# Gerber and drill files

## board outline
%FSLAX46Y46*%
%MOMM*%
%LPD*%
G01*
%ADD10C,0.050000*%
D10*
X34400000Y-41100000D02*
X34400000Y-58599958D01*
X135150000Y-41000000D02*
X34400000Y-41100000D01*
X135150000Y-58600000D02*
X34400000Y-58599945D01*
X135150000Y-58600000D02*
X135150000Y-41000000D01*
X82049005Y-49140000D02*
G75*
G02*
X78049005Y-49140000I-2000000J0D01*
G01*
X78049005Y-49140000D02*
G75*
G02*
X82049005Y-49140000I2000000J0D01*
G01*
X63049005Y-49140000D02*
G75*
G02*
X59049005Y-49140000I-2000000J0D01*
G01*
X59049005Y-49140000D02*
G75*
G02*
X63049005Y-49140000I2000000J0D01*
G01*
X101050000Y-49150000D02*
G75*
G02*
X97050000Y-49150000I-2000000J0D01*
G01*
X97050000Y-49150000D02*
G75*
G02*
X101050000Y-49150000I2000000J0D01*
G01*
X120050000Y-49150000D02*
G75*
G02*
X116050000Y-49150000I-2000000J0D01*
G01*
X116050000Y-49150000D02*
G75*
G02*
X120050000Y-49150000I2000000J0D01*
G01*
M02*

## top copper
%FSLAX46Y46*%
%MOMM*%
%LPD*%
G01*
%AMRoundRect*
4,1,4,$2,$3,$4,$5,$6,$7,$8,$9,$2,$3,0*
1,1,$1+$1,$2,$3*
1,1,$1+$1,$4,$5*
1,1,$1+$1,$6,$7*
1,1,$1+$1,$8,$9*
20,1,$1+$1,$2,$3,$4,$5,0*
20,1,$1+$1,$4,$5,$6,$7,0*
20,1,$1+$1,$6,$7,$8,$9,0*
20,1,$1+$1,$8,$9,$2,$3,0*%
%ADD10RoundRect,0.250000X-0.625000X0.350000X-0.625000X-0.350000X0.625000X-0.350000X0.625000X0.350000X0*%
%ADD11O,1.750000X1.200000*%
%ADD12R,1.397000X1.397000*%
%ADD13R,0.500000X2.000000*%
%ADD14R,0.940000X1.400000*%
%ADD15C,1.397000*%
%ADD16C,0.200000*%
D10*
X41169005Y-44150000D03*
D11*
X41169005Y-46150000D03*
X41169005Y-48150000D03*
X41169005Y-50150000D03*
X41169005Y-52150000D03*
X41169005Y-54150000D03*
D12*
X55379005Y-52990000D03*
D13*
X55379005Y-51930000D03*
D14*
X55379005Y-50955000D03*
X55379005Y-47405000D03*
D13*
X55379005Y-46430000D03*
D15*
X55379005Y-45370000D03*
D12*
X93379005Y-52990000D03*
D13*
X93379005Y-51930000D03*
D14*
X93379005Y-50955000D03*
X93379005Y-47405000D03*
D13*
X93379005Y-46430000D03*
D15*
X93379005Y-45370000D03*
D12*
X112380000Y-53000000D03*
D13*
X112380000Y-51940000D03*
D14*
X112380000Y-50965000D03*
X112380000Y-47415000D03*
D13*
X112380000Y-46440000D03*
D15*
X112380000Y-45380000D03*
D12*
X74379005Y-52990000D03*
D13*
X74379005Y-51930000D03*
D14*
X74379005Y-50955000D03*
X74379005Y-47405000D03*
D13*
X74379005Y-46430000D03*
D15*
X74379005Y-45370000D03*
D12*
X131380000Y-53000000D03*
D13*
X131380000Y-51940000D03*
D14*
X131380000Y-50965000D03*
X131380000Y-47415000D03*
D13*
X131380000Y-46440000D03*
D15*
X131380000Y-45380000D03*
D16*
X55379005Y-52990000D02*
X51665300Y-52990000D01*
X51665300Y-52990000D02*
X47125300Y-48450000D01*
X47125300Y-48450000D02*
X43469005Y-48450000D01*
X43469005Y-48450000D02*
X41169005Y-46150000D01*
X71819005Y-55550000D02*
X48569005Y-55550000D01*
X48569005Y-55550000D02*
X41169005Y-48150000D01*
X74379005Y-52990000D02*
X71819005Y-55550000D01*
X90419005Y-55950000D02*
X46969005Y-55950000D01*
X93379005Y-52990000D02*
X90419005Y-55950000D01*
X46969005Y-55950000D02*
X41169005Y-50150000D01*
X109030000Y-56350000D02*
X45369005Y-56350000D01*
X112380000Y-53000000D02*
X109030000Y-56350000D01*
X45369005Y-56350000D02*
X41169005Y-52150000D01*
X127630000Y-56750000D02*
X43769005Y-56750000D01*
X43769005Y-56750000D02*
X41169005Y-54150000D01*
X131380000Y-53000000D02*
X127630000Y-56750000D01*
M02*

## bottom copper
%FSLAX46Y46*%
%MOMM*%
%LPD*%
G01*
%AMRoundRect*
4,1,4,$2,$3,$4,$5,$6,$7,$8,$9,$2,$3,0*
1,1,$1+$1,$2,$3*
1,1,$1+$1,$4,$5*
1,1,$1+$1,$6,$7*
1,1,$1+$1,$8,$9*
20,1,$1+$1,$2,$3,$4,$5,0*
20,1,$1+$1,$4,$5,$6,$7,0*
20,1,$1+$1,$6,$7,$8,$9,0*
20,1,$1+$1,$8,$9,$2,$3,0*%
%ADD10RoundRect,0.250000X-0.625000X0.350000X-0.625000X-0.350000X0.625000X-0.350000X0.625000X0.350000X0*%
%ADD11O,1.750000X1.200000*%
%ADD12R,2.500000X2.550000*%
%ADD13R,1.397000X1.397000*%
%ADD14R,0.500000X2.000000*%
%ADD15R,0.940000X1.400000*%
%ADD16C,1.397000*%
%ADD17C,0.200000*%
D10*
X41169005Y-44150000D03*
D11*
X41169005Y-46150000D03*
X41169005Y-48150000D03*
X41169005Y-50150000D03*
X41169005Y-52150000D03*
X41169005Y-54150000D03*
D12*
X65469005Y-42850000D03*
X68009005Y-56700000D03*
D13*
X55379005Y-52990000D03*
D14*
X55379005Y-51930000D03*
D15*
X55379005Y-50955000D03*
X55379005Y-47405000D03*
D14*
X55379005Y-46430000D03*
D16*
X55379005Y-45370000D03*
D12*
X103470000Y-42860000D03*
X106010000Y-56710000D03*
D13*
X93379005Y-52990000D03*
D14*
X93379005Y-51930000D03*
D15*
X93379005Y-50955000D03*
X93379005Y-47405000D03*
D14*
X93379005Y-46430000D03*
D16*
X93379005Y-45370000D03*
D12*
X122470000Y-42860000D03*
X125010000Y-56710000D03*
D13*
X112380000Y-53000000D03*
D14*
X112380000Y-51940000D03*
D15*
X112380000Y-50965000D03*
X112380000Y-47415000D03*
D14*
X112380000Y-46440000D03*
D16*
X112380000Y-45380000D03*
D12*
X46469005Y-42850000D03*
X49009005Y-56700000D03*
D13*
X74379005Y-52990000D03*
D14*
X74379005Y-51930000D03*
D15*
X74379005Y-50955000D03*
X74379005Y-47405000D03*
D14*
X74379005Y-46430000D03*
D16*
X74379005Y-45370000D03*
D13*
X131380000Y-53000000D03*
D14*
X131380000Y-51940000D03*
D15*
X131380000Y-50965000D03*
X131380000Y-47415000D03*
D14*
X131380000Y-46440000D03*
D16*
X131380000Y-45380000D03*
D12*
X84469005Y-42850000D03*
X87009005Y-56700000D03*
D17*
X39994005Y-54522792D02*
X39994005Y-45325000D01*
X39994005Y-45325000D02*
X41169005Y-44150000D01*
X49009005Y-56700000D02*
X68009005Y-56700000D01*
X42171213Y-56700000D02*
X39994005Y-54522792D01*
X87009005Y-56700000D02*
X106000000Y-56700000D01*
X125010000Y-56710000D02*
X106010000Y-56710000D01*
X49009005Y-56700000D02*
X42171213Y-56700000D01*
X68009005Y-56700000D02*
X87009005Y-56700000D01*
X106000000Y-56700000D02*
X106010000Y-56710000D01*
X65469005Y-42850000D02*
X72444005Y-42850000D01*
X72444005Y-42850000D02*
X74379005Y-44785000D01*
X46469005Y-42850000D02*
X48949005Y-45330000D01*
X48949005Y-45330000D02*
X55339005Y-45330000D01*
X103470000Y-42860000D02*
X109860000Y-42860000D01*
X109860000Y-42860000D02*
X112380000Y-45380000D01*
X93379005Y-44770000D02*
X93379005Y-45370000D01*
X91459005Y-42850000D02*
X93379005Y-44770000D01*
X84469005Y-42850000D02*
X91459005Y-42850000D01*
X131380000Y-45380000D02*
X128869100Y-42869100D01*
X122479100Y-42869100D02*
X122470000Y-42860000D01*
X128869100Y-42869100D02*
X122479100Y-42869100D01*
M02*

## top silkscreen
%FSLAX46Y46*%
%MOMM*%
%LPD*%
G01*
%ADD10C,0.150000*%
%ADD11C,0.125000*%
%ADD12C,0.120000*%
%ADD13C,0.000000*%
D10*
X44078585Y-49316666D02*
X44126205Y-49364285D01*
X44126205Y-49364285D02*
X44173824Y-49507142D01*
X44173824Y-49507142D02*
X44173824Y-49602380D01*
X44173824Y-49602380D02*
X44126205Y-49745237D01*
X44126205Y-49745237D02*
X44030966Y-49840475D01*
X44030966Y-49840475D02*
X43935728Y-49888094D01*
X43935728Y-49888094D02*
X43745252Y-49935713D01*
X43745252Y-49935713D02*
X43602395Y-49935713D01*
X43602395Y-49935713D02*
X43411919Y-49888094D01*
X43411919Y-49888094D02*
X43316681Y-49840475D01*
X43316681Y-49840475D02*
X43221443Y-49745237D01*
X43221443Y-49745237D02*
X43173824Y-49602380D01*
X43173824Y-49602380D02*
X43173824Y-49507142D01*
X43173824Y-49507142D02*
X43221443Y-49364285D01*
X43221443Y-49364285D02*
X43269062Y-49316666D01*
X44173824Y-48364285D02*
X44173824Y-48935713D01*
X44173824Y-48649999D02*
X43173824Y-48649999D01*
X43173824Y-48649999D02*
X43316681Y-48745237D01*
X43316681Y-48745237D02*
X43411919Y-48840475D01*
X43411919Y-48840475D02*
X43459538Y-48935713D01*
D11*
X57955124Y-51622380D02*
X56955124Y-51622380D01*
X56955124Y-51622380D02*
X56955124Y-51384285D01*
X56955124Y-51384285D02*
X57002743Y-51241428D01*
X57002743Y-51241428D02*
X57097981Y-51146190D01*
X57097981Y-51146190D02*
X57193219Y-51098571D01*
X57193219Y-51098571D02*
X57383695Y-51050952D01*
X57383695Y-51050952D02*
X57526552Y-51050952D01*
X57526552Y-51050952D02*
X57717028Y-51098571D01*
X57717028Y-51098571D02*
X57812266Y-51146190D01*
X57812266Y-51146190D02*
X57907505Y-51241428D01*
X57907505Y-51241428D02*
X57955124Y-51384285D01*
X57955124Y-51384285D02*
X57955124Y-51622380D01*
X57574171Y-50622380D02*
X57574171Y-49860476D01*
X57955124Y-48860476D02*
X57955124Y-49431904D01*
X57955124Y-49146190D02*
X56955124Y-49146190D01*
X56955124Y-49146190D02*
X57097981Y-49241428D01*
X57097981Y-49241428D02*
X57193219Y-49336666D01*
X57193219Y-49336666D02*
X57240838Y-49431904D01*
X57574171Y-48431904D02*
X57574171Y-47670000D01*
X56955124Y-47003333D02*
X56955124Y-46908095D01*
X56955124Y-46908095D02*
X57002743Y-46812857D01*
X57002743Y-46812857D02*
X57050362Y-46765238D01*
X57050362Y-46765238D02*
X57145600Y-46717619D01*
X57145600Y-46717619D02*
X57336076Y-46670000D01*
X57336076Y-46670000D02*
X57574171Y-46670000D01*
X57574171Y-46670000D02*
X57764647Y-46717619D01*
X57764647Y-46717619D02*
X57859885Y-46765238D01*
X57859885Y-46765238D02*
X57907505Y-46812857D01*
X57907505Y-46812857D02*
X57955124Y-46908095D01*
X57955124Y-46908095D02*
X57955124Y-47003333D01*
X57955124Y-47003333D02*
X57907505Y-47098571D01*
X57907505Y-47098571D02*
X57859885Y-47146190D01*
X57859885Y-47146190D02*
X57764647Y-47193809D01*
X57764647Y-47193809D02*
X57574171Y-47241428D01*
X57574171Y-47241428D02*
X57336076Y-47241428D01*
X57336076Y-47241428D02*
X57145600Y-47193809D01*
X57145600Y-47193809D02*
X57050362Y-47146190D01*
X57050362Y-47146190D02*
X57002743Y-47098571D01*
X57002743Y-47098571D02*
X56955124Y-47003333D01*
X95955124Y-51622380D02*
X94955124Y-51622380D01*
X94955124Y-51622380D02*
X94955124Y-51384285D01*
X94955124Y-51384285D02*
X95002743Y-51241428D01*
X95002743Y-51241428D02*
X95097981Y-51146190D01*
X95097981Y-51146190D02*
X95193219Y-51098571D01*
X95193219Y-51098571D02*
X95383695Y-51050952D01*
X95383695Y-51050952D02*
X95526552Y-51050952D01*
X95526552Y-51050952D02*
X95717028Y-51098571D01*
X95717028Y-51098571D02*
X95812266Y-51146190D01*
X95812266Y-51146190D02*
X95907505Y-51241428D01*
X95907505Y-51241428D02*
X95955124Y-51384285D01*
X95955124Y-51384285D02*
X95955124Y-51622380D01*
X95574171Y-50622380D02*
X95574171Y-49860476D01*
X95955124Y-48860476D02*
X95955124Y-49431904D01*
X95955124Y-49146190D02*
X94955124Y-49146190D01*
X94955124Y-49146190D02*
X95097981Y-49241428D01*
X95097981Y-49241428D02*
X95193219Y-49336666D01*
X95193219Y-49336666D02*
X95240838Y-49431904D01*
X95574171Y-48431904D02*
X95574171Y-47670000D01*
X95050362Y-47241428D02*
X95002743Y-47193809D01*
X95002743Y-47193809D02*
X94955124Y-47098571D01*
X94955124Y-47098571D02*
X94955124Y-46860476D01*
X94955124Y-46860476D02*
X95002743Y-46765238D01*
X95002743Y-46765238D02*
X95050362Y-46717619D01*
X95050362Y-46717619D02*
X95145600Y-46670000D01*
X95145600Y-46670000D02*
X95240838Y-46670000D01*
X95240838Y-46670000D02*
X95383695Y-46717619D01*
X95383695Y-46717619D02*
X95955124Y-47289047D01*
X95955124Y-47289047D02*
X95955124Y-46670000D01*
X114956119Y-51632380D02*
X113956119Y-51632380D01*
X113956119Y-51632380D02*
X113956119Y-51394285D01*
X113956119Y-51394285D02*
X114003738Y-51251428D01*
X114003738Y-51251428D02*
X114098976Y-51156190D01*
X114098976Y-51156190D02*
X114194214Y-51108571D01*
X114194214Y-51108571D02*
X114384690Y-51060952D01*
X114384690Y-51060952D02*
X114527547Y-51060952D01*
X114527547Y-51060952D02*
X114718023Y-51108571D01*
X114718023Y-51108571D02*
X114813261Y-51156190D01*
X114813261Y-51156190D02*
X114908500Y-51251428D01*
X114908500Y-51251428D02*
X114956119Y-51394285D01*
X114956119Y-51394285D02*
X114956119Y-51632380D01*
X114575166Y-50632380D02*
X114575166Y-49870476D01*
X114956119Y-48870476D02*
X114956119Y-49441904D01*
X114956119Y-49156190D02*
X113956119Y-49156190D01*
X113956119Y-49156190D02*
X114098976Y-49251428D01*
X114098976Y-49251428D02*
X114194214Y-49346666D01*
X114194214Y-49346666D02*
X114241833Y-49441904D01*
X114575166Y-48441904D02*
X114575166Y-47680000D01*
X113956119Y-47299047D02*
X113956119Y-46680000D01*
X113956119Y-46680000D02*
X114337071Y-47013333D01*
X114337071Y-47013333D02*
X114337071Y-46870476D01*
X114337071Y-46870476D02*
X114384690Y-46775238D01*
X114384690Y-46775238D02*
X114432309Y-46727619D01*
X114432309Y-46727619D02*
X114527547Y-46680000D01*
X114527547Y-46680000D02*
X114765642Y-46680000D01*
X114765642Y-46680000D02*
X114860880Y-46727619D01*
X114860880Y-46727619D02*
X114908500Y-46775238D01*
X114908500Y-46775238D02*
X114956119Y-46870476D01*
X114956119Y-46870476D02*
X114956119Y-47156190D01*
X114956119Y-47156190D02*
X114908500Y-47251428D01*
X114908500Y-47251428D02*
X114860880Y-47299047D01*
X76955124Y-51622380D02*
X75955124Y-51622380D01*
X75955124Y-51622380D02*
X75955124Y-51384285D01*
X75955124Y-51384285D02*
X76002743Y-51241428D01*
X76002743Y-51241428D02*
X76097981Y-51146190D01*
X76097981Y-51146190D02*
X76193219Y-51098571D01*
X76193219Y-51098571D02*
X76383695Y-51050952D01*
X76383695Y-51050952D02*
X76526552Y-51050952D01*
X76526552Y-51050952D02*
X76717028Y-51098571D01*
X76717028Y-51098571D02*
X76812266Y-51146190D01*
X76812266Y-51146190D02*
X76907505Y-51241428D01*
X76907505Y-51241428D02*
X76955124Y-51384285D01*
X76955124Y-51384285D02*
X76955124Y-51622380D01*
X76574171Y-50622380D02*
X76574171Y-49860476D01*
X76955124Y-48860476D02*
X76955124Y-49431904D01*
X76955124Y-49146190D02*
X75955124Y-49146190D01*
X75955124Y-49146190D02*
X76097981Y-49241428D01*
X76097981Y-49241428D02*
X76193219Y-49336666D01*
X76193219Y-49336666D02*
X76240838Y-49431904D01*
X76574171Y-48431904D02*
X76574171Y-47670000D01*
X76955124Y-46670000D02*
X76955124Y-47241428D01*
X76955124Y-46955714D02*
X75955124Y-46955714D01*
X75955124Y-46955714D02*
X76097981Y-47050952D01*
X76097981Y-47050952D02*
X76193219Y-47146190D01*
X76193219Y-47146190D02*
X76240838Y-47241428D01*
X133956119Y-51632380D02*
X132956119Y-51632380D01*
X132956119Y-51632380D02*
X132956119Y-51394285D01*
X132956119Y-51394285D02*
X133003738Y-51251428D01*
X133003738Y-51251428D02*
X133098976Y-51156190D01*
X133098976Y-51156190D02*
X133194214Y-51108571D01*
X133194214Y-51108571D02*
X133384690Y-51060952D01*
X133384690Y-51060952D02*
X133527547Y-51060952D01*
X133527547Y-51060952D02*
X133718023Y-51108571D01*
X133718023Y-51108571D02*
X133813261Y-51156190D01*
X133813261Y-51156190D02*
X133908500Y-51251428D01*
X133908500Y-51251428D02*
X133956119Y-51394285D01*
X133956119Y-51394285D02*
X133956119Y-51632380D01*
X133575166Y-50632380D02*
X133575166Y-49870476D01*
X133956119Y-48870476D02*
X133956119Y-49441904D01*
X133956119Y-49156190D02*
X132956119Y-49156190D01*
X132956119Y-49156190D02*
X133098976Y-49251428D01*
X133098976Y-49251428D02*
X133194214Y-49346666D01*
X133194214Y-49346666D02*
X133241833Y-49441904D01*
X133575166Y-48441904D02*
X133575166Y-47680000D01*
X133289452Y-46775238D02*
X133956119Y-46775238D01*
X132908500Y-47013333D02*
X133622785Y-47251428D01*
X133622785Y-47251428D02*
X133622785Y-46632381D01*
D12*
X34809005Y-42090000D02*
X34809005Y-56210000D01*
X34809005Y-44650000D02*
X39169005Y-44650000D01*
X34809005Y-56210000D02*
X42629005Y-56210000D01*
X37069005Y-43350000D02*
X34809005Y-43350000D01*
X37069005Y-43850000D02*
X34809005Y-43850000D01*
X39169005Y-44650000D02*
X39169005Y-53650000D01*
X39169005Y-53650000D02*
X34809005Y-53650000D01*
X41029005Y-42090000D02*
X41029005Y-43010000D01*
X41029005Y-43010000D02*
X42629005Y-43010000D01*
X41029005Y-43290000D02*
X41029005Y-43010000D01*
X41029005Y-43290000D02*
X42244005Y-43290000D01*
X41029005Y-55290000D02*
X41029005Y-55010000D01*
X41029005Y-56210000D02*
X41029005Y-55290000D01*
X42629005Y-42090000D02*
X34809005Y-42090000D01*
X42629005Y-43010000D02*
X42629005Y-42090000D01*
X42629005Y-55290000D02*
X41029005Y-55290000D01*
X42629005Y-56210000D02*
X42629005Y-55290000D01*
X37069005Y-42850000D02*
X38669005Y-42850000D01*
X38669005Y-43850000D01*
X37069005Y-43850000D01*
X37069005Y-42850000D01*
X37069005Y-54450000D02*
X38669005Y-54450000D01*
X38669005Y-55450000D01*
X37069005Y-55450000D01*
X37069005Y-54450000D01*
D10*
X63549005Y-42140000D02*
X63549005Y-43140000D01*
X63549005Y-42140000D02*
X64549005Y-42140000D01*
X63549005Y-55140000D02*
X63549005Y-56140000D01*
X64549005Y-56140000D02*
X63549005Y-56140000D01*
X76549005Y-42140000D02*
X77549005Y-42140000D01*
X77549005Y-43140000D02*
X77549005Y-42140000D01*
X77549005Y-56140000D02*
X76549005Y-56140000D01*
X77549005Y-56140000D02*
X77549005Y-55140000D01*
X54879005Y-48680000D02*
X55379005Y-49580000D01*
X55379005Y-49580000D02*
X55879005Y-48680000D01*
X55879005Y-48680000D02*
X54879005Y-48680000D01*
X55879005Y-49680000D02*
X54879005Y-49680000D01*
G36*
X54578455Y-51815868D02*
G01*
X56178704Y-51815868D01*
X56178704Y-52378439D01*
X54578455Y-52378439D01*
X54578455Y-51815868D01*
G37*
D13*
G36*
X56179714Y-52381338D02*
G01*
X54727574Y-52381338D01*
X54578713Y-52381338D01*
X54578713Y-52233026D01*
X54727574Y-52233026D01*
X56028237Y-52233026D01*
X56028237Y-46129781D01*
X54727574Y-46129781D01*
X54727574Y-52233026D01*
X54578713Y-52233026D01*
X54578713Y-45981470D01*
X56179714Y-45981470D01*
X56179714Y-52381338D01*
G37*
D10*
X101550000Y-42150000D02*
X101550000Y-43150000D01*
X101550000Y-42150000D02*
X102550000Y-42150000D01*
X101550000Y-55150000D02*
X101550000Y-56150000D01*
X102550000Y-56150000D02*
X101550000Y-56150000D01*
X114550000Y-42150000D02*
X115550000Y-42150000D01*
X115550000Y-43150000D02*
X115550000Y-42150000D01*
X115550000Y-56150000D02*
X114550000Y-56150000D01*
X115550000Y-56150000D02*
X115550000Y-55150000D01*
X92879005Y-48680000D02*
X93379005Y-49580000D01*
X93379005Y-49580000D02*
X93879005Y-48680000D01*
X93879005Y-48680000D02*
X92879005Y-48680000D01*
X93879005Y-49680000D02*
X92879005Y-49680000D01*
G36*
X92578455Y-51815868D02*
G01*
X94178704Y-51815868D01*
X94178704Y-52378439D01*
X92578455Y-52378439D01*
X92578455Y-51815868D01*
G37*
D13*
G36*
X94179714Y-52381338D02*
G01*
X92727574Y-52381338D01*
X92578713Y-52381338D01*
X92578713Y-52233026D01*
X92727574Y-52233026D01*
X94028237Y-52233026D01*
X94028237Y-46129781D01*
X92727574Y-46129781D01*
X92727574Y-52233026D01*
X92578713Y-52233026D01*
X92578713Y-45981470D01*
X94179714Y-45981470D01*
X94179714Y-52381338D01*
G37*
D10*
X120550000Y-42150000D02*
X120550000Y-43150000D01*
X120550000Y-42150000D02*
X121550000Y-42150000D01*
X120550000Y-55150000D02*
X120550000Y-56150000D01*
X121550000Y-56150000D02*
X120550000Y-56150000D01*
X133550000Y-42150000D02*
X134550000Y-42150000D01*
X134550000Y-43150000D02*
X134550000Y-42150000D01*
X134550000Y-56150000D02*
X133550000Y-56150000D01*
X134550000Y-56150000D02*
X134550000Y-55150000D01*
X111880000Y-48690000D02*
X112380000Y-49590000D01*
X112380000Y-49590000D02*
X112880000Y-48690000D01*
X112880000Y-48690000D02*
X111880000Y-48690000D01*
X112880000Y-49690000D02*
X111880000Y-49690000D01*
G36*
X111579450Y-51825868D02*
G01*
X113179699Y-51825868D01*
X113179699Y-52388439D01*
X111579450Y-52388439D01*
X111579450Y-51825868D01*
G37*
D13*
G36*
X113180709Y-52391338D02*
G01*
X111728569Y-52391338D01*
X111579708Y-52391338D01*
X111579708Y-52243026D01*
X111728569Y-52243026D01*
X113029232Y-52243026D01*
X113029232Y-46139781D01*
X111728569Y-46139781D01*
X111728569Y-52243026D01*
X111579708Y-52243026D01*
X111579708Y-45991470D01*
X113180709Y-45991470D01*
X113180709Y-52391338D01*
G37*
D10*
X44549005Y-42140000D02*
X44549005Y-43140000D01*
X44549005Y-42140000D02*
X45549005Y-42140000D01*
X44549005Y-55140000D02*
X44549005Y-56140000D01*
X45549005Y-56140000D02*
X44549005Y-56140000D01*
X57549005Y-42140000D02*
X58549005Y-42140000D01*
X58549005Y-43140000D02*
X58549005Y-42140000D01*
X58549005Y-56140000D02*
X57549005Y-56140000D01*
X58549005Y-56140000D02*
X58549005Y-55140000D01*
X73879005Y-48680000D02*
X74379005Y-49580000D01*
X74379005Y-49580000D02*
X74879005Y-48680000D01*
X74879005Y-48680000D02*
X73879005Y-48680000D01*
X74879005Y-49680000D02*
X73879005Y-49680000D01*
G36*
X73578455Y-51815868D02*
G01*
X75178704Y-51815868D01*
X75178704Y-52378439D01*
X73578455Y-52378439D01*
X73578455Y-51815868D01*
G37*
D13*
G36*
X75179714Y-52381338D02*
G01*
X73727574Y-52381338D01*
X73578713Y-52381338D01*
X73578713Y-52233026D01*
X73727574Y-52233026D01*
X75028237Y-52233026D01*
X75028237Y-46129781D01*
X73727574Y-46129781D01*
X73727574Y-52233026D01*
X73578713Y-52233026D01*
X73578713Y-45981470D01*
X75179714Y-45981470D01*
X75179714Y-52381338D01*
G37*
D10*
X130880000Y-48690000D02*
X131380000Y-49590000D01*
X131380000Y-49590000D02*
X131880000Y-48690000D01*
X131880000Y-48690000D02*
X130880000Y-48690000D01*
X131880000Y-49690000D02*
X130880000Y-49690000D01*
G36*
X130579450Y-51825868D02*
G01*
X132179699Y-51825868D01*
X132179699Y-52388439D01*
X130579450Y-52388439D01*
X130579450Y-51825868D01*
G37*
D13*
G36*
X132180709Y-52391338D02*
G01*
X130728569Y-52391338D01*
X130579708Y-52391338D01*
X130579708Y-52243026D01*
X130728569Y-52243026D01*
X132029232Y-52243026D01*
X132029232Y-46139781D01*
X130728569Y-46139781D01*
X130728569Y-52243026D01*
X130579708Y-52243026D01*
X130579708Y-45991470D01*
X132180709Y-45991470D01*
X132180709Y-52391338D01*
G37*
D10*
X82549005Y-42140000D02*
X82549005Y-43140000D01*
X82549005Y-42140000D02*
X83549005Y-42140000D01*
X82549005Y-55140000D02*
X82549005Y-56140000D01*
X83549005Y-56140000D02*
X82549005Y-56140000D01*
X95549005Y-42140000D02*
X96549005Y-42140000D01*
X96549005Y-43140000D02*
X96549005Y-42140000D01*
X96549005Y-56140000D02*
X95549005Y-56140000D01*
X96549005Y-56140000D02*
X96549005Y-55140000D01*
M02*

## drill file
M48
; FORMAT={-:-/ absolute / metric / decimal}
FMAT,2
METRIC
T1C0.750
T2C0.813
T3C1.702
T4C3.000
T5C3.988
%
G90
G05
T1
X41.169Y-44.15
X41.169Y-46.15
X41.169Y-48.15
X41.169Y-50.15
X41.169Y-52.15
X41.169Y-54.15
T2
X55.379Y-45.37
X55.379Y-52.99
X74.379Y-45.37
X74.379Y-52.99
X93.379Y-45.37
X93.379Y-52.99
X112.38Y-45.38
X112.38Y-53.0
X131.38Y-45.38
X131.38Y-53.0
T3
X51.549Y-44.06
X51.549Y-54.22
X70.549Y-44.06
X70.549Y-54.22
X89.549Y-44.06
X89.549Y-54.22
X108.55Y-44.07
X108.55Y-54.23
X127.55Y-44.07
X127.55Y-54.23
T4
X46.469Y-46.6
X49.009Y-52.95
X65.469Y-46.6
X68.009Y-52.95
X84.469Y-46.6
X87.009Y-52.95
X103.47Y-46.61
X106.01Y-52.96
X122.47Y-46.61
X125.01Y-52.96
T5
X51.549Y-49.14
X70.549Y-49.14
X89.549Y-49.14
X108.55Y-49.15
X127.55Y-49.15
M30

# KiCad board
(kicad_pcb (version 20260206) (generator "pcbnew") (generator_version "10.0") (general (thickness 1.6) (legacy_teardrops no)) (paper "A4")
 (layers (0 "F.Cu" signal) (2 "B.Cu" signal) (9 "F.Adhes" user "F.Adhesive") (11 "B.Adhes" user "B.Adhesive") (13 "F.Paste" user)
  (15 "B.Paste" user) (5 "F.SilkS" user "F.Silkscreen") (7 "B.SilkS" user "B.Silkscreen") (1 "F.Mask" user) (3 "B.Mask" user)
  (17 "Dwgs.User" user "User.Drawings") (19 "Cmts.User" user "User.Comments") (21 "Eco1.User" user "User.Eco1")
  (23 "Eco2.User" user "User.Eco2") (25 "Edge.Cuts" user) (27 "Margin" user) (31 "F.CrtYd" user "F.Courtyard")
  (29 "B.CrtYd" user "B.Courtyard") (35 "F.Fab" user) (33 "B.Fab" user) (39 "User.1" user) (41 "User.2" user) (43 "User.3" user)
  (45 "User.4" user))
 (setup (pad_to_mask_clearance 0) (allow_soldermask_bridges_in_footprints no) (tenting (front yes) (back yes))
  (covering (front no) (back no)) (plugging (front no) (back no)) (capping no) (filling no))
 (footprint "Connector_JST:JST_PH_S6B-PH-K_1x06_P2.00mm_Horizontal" (layer "F.Cu") (at 41.169005 44.15 -90)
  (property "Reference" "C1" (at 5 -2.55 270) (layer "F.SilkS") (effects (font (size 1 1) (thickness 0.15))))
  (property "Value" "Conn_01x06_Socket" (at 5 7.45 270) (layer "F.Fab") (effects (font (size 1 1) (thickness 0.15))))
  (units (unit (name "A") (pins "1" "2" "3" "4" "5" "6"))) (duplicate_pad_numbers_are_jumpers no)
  (fp_line (start -2.06 6.36) (end 12.06 6.36) (stroke (width 0.12) (type solid)) (layer "F.SilkS"))
  (fp_line (start 0.5 6.36) (end 0.5 2) (stroke (width 0.12) (type solid)) (layer "F.SilkS"))
  (fp_line (start 12.06 6.36) (end 12.06 -1.46) (stroke (width 0.12) (type solid)) (layer "F.SilkS"))
  (fp_line (start -0.8 4.1) (end -0.8 6.36) (stroke (width 0.12) (type solid)) (layer "F.SilkS"))
  (fp_line (start -0.3 4.1) (end -0.3 6.36) (stroke (width 0.12) (type solid)) (layer "F.SilkS"))
  (fp_line (start 0.5 2) (end 9.5 2) (stroke (width 0.12) (type solid)) (layer "F.SilkS"))
  (fp_line (start 9.5 2) (end 9.5 6.36) (stroke (width 0.12) (type solid)) (layer "F.SilkS"))
  (fp_line (start -2.06 0.14) (end -1.14 0.14) (stroke (width 0.12) (type solid)) (layer "F.SilkS"))
  (fp_line (start -1.14 0.14) (end -1.14 -1.46) (stroke (width 0.12) (type solid)) (layer "F.SilkS"))
  (fp_line (start -0.86 0.14) (end -1.14 0.14) (stroke (width 0.12) (type solid)) (layer "F.SilkS"))
  (fp_line (start -0.86 0.14) (end -0.86 -1.075) (stroke (width 0.12) (type solid)) (layer "F.SilkS"))
  (fp_line (start 11.14 0.14) (end 10.86 0.14) (stroke (width 0.12) (type solid)) (layer "F.SilkS"))
  (fp_line (start 12.06 0.14) (end 11.14 0.14) (stroke (width 0.12) (type solid)) (layer "F.SilkS"))
  (fp_line (start -2.06 -1.46) (end -2.06 6.36) (stroke (width 0.12) (type solid)) (layer "F.SilkS"))
  (fp_line (start -1.14 -1.46) (end -2.06 -1.46) (stroke (width 0.12) (type solid)) (layer "F.SilkS"))
  (fp_line (start 11.14 -1.46) (end 11.14 0.14) (stroke (width 0.12) (type solid)) (layer "F.SilkS"))
  (fp_line (start 12.06 -1.46) (end 11.14 -1.46) (stroke (width 0.12) (type solid)) (layer "F.SilkS"))
  (fp_rect (start -1.3 2.5) (end -0.3 4.1) (stroke (width 0.12) (type solid)) (fill no) (layer "F.SilkS"))
  (fp_rect (start 10.3 2.5) (end 11.3 4.1) (stroke (width 0.12) (type solid)) (fill no) (layer "F.SilkS"))
  (pad "1" thru_hole roundrect (at 0 0 270) (size 1.2 1.75) (drill 0.75) (layers "*.Cu" "*.Mask") (remove_unused_layers no)
   (roundrect_rratio 0.208333) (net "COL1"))
  (pad "2" thru_hole oval (at 2 0 270) (size 1.2 1.75) (drill 0.75) (layers "*.Cu" "*.Mask") (remove_unused_layers no) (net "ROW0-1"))
  (pad "3" thru_hole oval (at 4 0 270) (size 1.2 1.75) (drill 0.75) (layers "*.Cu" "*.Mask") (remove_unused_layers no) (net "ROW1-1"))
  (pad "4" thru_hole oval (at 6 0 270) (size 1.2 1.75) (drill 0.75) (layers "*.Cu" "*.Mask") (remove_unused_layers no) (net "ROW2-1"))
  (pad "5" thru_hole oval (at 8 0 270) (size 1.2 1.75) (drill 0.75) (layers "*.Cu" "*.Mask") (remove_unused_layers no) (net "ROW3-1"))
  (pad "6" thru_hole oval (at 10 0 270) (size 1.2 1.75) (drill 0.75) (layers "*.Cu" "*.Mask") (remove_unused_layers no) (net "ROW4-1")))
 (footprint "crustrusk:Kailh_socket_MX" (layer "F.Cu") (at 70.549005 49.14 90)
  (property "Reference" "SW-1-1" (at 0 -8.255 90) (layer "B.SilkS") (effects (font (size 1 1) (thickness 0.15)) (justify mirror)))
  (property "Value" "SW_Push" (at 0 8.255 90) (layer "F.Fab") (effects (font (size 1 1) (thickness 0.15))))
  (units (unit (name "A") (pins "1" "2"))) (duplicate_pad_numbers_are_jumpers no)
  (fp_line (start 7 -7) (end 6 -7) (stroke (width 0.15) (type solid)) (layer "F.SilkS"))
  (fp_line (start 7 -7) (end 7 -6) (stroke (width 0.15) (type solid)) (layer "F.SilkS"))
  (fp_line (start -6 -7) (end -7 -7) (stroke (width 0.15) (type solid)) (layer "F.SilkS"))
  (fp_line (start -7 -6) (end -7 -7) (stroke (width 0.15) (type solid)) (layer "F.SilkS"))
  (fp_line (start 7 6) (end 7 7) (stroke (width 0.15) (type solid)) (layer "F.SilkS"))
  (fp_line (start 6 7) (end 7 7) (stroke (width 0.15) (type solid)) (layer "F.SilkS"))
  (fp_line (start -7 7) (end -7 6) (stroke (width 0.15) (type solid)) (layer "F.SilkS"))
  (fp_line (start -7 7) (end -6 7) (stroke (width 0.15) (type solid)) (layer "F.SilkS"))
  (pad "" np_thru_hole circle (at -5.08 0 90) (size 1.7018 1.7018) (drill 1.7018) (layers "*.Cu" "*.Mask"))
  (pad "" np_thru_hole circle (at -3.81 -2.54 90) (size 3 3) (drill 3) (layers "*.Cu" "*.Mask"))
  (pad "" np_thru_hole circle (at 0 0 90) (size 3.9878 3.9878) (drill 3.9878) (layers "*.Cu" "*.Mask"))
  (pad "" np_thru_hole circle (at 2.54 -5.08 90) (size 3 3) (drill 3) (layers "*.Cu" "*.Mask"))
  (pad "" np_thru_hole circle (at 5.08 0 90) (size 1.7018 1.7018) (drill 1.7018) (layers "*.Cu" "*.Mask"))
  (pad "1" smd rect (at 6.29 -5.08 90) (size 2.55 2.5) (layers "B.Cu" "B.Mask" "B.Paste") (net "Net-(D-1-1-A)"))
  (pad "2" smd rect (at -7.56 -2.54 90) (size 2.55 2.5) (layers "B.Cu" "B.Mask" "B.Paste") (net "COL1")))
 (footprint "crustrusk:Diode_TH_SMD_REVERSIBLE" (layer "F.Cu") (at 55.379005 49.18 90)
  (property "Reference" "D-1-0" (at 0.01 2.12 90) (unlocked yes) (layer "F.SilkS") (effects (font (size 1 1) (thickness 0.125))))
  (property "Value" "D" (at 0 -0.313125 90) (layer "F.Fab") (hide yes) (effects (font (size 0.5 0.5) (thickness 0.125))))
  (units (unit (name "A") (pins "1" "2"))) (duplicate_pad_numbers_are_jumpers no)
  (fp_line (start 0.5 -0.5) (end -0.4 0) (stroke (width 0.15) (type solid)) (layer "F.SilkS"))
  (fp_line (start -0.4 0) (end 0.5 0.5) (stroke (width 0.15) (type solid)) (layer "F.SilkS"))
  (fp_line (start 0.5 0.5) (end 0.5 -0.5) (stroke (width 0.15) (type solid)) (layer "F.SilkS"))
  (fp_line (start -0.5 0.5) (end -0.5 -0.5) (stroke (width 0.15) (type solid)) (layer "F.SilkS"))
  (fp_rect (start -3.198439 -0.80055) (end -2.635868 0.799699) (stroke (width -0.000001) (type solid)) (fill yes) (layer "F.SilkS"))
  (fp_poly
   (pts (xy 3.19853 -0.800292) (xy -3.201338 -0.800292) (xy -3.201338 -0.651431) (xy -3.053026 -0.651431) (xy 3.050219 -0.651431)
    (xy 3.050219 0.649232) (xy -3.053026 0.649232) (xy -3.053026 -0.651431) (xy -3.201338 -0.651431) (xy -3.201338 0.800709)
    (xy 3.19853 0.800709))
   (stroke (width -0.000001) (type solid)) (fill yes) (layer "F.SilkS"))
  (pad "1" thru_hole rect (at -3.81 0 90) (size 1.397 1.397) (drill 0.8128) (layers "*.Cu" "*.Mask") (remove_unused_layers no)
   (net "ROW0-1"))
  (pad "1" smd rect (at -2.75 0 270) (size 2 0.5) (layers "F.Cu") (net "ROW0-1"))
  (pad "1" smd rect (at -2.75 0 90) (size 2 0.5) (layers "B.Cu") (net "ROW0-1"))
  (pad "1" smd rect (at -1.775 0 270) (size 1.4 0.94) (layers "F.Cu" "F.Mask" "F.Paste") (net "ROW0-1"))
  (pad "1" smd rect (at -1.775 0 90) (size 1.4 0.94) (layers "B.Cu" "B.Mask" "B.Paste") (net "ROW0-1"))
  (pad "2" smd rect (at 1.775 0 270) (size 1.4 0.94) (layers "F.Cu" "F.Mask" "F.Paste") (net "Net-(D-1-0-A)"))
  (pad "2" smd rect (at 1.775 0 90) (size 1.4 0.94) (layers "B.Cu" "B.Mask" "B.Paste") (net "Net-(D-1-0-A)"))
  (pad "2" smd rect (at 2.75 0 270) (size 2 0.5) (layers "F.Cu") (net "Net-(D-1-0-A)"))
  (pad "2" smd rect (at 2.75 0 90) (size 2 0.5) (layers "B.Cu") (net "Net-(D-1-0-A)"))
  (pad "2" thru_hole circle (at 3.81 0 90) (size 1.397 1.397) (drill 0.8128) (layers "*.Cu" "*.Mask") (remove_unused_layers no)
   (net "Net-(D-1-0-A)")))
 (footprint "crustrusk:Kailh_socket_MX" (layer "F.Cu") (at 108.55 49.15 90)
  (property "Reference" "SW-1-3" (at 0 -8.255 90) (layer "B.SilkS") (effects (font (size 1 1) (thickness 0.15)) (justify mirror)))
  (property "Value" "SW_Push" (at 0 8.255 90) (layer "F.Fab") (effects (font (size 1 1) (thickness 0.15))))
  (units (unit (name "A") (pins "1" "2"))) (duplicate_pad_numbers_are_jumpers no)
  (fp_line (start 7 -7) (end 6 -7) (stroke (width 0.15) (type solid)) (layer "F.SilkS"))
  (fp_line (start 7 -7) (end 7 -6) (stroke (width 0.15) (type solid)) (layer "F.SilkS"))
  (fp_line (start -6 -7) (end -7 -7) (stroke (width 0.15) (type solid)) (layer "F.SilkS"))
  (fp_line (start -7 -6) (end -7 -7) (stroke (width 0.15) (type solid)) (layer "F.SilkS"))
  (fp_line (start 7 6) (end 7 7) (stroke (width 0.15) (type solid)) (layer "F.SilkS"))
  (fp_line (start 6 7) (end 7 7) (stroke (width 0.15) (type solid)) (layer "F.SilkS"))
  (fp_line (start -7 7) (end -7 6) (stroke (width 0.15) (type solid)) (layer "F.SilkS"))
  (fp_line (start -7 7) (end -6 7) (stroke (width 0.15) (type solid)) (layer "F.SilkS"))
  (pad "" np_thru_hole circle (at -5.08 0 90) (size 1.7018 1.7018) (drill 1.7018) (layers "*.Cu" "*.Mask"))
  (pad "" np_thru_hole circle (at -3.81 -2.54 90) (size 3 3) (drill 3) (layers "*.Cu" "*.Mask"))
  (pad "" np_thru_hole circle (at 0 0 90) (size 3.9878 3.9878) (drill 3.9878) (layers "*.Cu" "*.Mask"))
  (pad "" np_thru_hole circle (at 2.54 -5.08 90) (size 3 3) (drill 3) (layers "*.Cu" "*.Mask"))
  (pad "" np_thru_hole circle (at 5.08 0 90) (size 1.7018 1.7018) (drill 1.7018) (layers "*.Cu" "*.Mask"))
  (pad "1" smd rect (at 6.29 -5.08 90) (size 2.55 2.5) (layers "B.Cu" "B.Mask" "B.Paste") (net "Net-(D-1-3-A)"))
  (pad "2" smd rect (at -7.56 -2.54 90) (size 2.55 2.5) (layers "B.Cu" "B.Mask" "B.Paste") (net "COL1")))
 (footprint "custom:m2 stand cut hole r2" (layer "F.Cu") (at 80.049005 49.14 90)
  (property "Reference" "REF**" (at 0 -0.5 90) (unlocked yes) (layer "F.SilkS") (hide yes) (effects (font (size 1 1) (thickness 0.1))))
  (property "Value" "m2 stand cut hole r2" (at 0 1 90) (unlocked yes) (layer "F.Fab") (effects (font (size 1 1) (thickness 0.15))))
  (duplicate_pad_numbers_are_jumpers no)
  (fp_circle (center 0 0) (end 2 0) (stroke (width 0.05) (type default)) (fill no) (layer "Edge.Cuts")))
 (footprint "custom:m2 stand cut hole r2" (layer "F.Cu") (at 61.049005 49.14 90)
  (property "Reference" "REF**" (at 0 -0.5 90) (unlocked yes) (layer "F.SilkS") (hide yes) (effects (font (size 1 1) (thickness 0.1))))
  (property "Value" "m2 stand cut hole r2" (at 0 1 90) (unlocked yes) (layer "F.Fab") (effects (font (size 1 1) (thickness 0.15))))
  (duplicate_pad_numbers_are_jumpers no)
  (fp_circle (center 0 0) (end 2 0) (stroke (width 0.05) (type default)) (fill no) (layer "Edge.Cuts")))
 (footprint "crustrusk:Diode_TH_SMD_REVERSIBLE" (layer "F.Cu") (at 93.379005 49.18 90)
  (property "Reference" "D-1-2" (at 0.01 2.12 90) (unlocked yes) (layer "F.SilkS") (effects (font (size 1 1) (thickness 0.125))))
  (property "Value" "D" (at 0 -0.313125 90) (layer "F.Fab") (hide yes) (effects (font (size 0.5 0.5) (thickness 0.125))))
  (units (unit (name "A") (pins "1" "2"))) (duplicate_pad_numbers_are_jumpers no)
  (fp_line (start 0.5 -0.5) (end -0.4 0) (stroke (width 0.15) (type solid)) (layer "F.SilkS"))
  (fp_line (start -0.4 0) (end 0.5 0.5) (stroke (width 0.15) (type solid)) (layer "F.SilkS"))
  (fp_line (start 0.5 0.5) (end 0.5 -0.5) (stroke (width 0.15) (type solid)) (layer "F.SilkS"))
  (fp_line (start -0.5 0.5) (end -0.5 -0.5) (stroke (width 0.15) (type solid)) (layer "F.SilkS"))
  (fp_rect (start -3.198439 -0.80055) (end -2.635868 0.799699) (stroke (width -0.000001) (type solid)) (fill yes) (layer "F.SilkS"))
  (fp_poly
   (pts (xy 3.19853 -0.800292) (xy -3.201338 -0.800292) (xy -3.201338 -0.651431) (xy -3.053026 -0.651431) (xy 3.050219 -0.651431)
    (xy 3.050219 0.649232) (xy -3.053026 0.649232) (xy -3.053026 -0.651431) (xy -3.201338 -0.651431) (xy -3.201338 0.800709)
    (xy 3.19853 0.800709))
   (stroke (width -0.000001) (type solid)) (fill yes) (layer "F.SilkS"))
  (pad "1" thru_hole rect (at -3.81 0 90) (size 1.397 1.397) (drill 0.8128) (layers "*.Cu" "*.Mask") (remove_unused_layers no)
   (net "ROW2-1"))
  (pad "1" smd rect (at -2.75 0 270) (size 2 0.5) (layers "F.Cu") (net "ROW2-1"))
  (pad "1" smd rect (at -2.75 0 90) (size 2 0.5) (layers "B.Cu") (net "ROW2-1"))
  (pad "1" smd rect (at -1.775 0 270) (size 1.4 0.94) (layers "F.Cu" "F.Mask" "F.Paste") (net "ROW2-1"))
  (pad "1" smd rect (at -1.775 0 90) (size 1.4 0.94) (layers "B.Cu" "B.Mask" "B.Paste") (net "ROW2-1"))
  (pad "2" smd rect (at 1.775 0 270) (size 1.4 0.94) (layers "F.Cu" "F.Mask" "F.Paste") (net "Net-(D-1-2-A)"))
  (pad "2" smd rect (at 1.775 0 90) (size 1.4 0.94) (layers "B.Cu" "B.Mask" "B.Paste") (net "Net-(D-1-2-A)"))
  (pad "2" smd rect (at 2.75 0 270) (size 2 0.5) (layers "F.Cu") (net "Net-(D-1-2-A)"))
  (pad "2" smd rect (at 2.75 0 90) (size 2 0.5) (layers "B.Cu") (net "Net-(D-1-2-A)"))
  (pad "2" thru_hole circle (at 3.81 0 90) (size 1.397 1.397) (drill 0.8128) (layers "*.Cu" "*.Mask") (remove_unused_layers no)
   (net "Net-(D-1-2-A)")))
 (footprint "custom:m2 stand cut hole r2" (layer "F.Cu") (at 99.05 49.15 90)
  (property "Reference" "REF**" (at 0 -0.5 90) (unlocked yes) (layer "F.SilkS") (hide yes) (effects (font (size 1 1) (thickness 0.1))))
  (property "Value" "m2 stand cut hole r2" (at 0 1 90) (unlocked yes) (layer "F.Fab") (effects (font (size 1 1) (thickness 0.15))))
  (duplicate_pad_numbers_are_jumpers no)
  (fp_circle (center 0 0) (end 2 0) (stroke (width 0.05) (type default)) (fill no) (layer "Edge.Cuts")))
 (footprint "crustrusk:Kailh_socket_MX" (layer "F.Cu") (at 127.55 49.15 90)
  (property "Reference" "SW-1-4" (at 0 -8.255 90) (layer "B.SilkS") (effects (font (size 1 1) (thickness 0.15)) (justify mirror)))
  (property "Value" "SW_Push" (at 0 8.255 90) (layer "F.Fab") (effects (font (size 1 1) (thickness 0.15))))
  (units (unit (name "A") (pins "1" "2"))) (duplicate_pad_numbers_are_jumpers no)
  (fp_line (start 7 -7) (end 6 -7) (stroke (width 0.15) (type solid)) (layer "F.SilkS"))
  (fp_line (start 7 -7) (end 7 -6) (stroke (width 0.15) (type solid)) (layer "F.SilkS"))
  (fp_line (start -6 -7) (end -7 -7) (stroke (width 0.15) (type solid)) (layer "F.SilkS"))
  (fp_line (start -7 -6) (end -7 -7) (stroke (width 0.15) (type solid)) (layer "F.SilkS"))
  (fp_line (start 7 6) (end 7 7) (stroke (width 0.15) (type solid)) (layer "F.SilkS"))
  (fp_line (start 6 7) (end 7 7) (stroke (width 0.15) (type solid)) (layer "F.SilkS"))
  (fp_line (start -7 7) (end -7 6) (stroke (width 0.15) (type solid)) (layer "F.SilkS"))
  (fp_line (start -7 7) (end -6 7) (stroke (width 0.15) (type solid)) (layer "F.SilkS"))
  (pad "" np_thru_hole circle (at -5.08 0 90) (size 1.7018 1.7018) (drill 1.7018) (layers "*.Cu" "*.Mask"))
  (pad "" np_thru_hole circle (at -3.81 -2.54 90) (size 3 3) (drill 3) (layers "*.Cu" "*.Mask"))
  (pad "" np_thru_hole circle (at 0 0 90) (size 3.9878 3.9878) (drill 3.9878) (layers "*.Cu" "*.Mask"))
  (pad "" np_thru_hole circle (at 2.54 -5.08 90) (size 3 3) (drill 3) (layers "*.Cu" "*.Mask"))
  (pad "" np_thru_hole circle (at 5.08 0 90) (size 1.7018 1.7018) (drill 1.7018) (layers "*.Cu" "*.Mask"))
  (pad "1" smd rect (at 6.29 -5.08 90) (size 2.55 2.5) (layers "B.Cu" "B.Mask" "B.Paste") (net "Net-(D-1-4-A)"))
  (pad "2" smd rect (at -7.56 -2.54 90) (size 2.55 2.5) (layers "B.Cu" "B.Mask" "B.Paste") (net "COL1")))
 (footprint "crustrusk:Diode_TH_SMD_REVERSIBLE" (layer "F.Cu") (at 112.38 49.19 90)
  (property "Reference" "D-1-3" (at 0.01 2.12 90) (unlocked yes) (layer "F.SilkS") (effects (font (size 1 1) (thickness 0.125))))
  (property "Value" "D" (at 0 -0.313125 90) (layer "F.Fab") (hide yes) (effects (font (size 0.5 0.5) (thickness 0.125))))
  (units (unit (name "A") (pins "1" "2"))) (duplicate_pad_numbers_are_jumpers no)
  (fp_line (start 0.5 -0.5) (end -0.4 0) (stroke (width 0.15) (type solid)) (layer "F.SilkS"))
  (fp_line (start -0.4 0) (end 0.5 0.5) (stroke (width 0.15) (type solid)) (layer "F.SilkS"))
  (fp_line (start 0.5 0.5) (end 0.5 -0.5) (stroke (width 0.15) (type solid)) (layer "F.SilkS"))
  (fp_line (start -0.5 0.5) (end -0.5 -0.5) (stroke (width 0.15) (type solid)) (layer "F.SilkS"))
  (fp_rect (start -3.198439 -0.80055) (end -2.635868 0.799699) (stroke (width -0.000001) (type solid)) (fill yes) (layer "F.SilkS"))
  (fp_poly
   (pts (xy 3.19853 -0.800292) (xy -3.201338 -0.800292) (xy -3.201338 -0.651431) (xy -3.053026 -0.651431) (xy 3.050219 -0.651431)
    (xy 3.050219 0.649232) (xy -3.053026 0.649232) (xy -3.053026 -0.651431) (xy -3.201338 -0.651431) (xy -3.201338 0.800709)
    (xy 3.19853 0.800709))
   (stroke (width -0.000001) (type solid)) (fill yes) (layer "F.SilkS"))
  (pad "1" thru_hole rect (at -3.81 0 90) (size 1.397 1.397) (drill 0.8128) (layers "*.Cu" "*.Mask") (remove_unused_layers no)
   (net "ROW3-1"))
  (pad "1" smd rect (at -2.75 0 270) (size 2 0.5) (layers "F.Cu") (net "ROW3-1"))
  (pad "1" smd rect (at -2.75 0 90) (size 2 0.5) (layers "B.Cu") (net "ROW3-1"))
  (pad "1" smd rect (at -1.775 0 270) (size 1.4 0.94) (layers "F.Cu" "F.Mask" "F.Paste") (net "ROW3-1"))
  (pad "1" smd rect (at -1.775 0 90) (size 1.4 0.94) (layers "B.Cu" "B.Mask" "B.Paste") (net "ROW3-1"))
  (pad "2" smd rect (at 1.775 0 270) (size 1.4 0.94) (layers "F.Cu" "F.Mask" "F.Paste") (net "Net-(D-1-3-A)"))
  (pad "2" smd rect (at 1.775 0 90) (size 1.4 0.94) (layers "B.Cu" "B.Mask" "B.Paste") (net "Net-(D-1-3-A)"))
  (pad "2" smd rect (at 2.75 0 270) (size 2 0.5) (layers "F.Cu") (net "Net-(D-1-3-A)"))
  (pad "2" smd rect (at 2.75 0 90) (size 2 0.5) (layers "B.Cu") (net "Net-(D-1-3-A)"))
  (pad "2" thru_hole circle (at 3.81 0 90) (size 1.397 1.397) (drill 0.8128) (layers "*.Cu" "*.Mask") (remove_unused_layers no)
   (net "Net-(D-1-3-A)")))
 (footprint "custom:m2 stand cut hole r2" (layer "F.Cu") (at 118.05 49.15 90)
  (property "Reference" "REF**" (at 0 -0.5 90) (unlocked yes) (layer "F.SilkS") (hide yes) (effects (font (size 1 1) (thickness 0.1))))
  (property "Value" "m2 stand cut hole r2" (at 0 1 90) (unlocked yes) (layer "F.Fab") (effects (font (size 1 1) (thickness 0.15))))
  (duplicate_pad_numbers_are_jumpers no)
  (fp_circle (center 0 0) (end 2 0) (stroke (width 0.05) (type default)) (fill no) (layer "Edge.Cuts")))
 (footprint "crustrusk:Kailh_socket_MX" (layer "F.Cu") (at 51.549005 49.14 90)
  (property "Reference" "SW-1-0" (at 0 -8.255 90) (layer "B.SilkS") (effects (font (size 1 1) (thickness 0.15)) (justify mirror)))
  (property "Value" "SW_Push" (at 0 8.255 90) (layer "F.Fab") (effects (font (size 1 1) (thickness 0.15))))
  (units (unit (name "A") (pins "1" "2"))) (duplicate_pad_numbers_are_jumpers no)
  (fp_line (start 7 -7) (end 6 -7) (stroke (width 0.15) (type solid)) (layer "F.SilkS"))
  (fp_line (start 7 -7) (end 7 -6) (stroke (width 0.15) (type solid)) (layer "F.SilkS"))
  (fp_line (start -6 -7) (end -7 -7) (stroke (width 0.15) (type solid)) (layer "F.SilkS"))
  (fp_line (start -7 -6) (end -7 -7) (stroke (width 0.15) (type solid)) (layer "F.SilkS"))
  (fp_line (start 7 6) (end 7 7) (stroke (width 0.15) (type solid)) (layer "F.SilkS"))
  (fp_line (start 6 7) (end 7 7) (stroke (width 0.15) (type solid)) (layer "F.SilkS"))
  (fp_line (start -7 7) (end -7 6) (stroke (width 0.15) (type solid)) (layer "F.SilkS"))
  (fp_line (start -7 7) (end -6 7) (stroke (width 0.15) (type solid)) (layer "F.SilkS"))
  (pad "" np_thru_hole circle (at -5.08 0 90) (size 1.7018 1.7018) (drill 1.7018) (layers "*.Cu" "*.Mask"))
  (pad "" np_thru_hole circle (at -3.81 -2.54 90) (size 3 3) (drill 3) (layers "*.Cu" "*.Mask"))
  (pad "" np_thru_hole circle (at 0 0 90) (size 3.9878 3.9878) (drill 3.9878) (layers "*.Cu" "*.Mask"))
  (pad "" np_thru_hole circle (at 2.54 -5.08 90) (size 3 3) (drill 3) (layers "*.Cu" "*.Mask"))
  (pad "" np_thru_hole circle (at 5.08 0 90) (size 1.7018 1.7018) (drill 1.7018) (layers "*.Cu" "*.Mask"))
  (pad "1" smd rect (at 6.29 -5.08 90) (size 2.55 2.5) (layers "B.Cu" "B.Mask" "B.Paste") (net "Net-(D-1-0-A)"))
  (pad "2" smd rect (at -7.56 -2.54 90) (size 2.55 2.5) (layers "B.Cu" "B.Mask" "B.Paste") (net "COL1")))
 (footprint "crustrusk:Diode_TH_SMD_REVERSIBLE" (layer "F.Cu") (at 74.379005 49.18 90)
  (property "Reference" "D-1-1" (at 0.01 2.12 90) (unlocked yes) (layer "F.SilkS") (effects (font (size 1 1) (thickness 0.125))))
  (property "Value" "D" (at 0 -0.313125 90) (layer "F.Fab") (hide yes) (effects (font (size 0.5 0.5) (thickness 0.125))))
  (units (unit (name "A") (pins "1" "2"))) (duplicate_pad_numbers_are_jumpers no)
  (fp_line (start 0.5 -0.5) (end -0.4 0) (stroke (width 0.15) (type solid)) (layer "F.SilkS"))
  (fp_line (start -0.4 0) (end 0.5 0.5) (stroke (width 0.15) (type solid)) (layer "F.SilkS"))
  (fp_line (start 0.5 0.5) (end 0.5 -0.5) (stroke (width 0.15) (type solid)) (layer "F.SilkS"))
  (fp_line (start -0.5 0.5) (end -0.5 -0.5) (stroke (width 0.15) (type solid)) (layer "F.SilkS"))
  (fp_rect (start -3.198439 -0.80055) (end -2.635868 0.799699) (stroke (width -0.000001) (type solid)) (fill yes) (layer "F.SilkS"))
  (fp_poly
   (pts (xy 3.19853 -0.800292) (xy -3.201338 -0.800292) (xy -3.201338 -0.651431) (xy -3.053026 -0.651431) (xy 3.050219 -0.651431)
    (xy 3.050219 0.649232) (xy -3.053026 0.649232) (xy -3.053026 -0.651431) (xy -3.201338 -0.651431) (xy -3.201338 0.800709)
    (xy 3.19853 0.800709))
   (stroke (width -0.000001) (type solid)) (fill yes) (layer "F.SilkS"))
  (pad "1" thru_hole rect (at -3.81 0 90) (size 1.397 1.397) (drill 0.8128) (layers "*.Cu" "*.Mask") (remove_unused_layers no)
   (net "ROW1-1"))
  (pad "1" smd rect (at -2.75 0 270) (size 2 0.5) (layers "F.Cu") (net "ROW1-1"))
  (pad "1" smd rect (at -2.75 0 90) (size 2 0.5) (layers "B.Cu") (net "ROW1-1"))
  (pad "1" smd rect (at -1.775 0 270) (size 1.4 0.94) (layers "F.Cu" "F.Mask" "F.Paste") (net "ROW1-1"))
  (pad "1" smd rect (at -1.775 0 90) (size 1.4 0.94) (layers "B.Cu" "B.Mask" "B.Paste") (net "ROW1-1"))
  (pad "2" smd rect (at 1.775 0 270) (size 1.4 0.94) (layers "F.Cu" "F.Mask" "F.Paste") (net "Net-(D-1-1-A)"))
  (pad "2" smd rect (at 1.775 0 90) (size 1.4 0.94) (layers "B.Cu" "B.Mask" "B.Paste") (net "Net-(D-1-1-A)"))
  (pad "2" smd rect (at 2.75 0 270) (size 2 0.5) (layers "F.Cu") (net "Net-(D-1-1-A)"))
  (pad "2" smd rect (at 2.75 0 90) (size 2 0.5) (layers "B.Cu") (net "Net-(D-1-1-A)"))
  (pad "2" thru_hole circle (at 3.81 0 90) (size 1.397 1.397) (drill 0.8128) (layers "*.Cu" "*.Mask") (remove_unused_layers no)
   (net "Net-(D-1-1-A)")))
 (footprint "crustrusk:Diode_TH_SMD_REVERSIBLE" (layer "F.Cu") (at 131.38 49.19 90)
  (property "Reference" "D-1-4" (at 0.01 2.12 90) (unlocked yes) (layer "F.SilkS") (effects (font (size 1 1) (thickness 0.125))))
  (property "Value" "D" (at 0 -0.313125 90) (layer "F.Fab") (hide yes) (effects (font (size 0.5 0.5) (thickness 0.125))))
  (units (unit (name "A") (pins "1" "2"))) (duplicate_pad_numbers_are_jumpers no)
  (fp_line (start 0.5 -0.5) (end -0.4 0) (stroke (width 0.15) (type solid)) (layer "F.SilkS"))
  (fp_line (start -0.4 0) (end 0.5 0.5) (stroke (width 0.15) (type solid)) (layer "F.SilkS"))
  (fp_line (start 0.5 0.5) (end 0.5 -0.5) (stroke (width 0.15) (type solid)) (layer "F.SilkS"))
  (fp_line (start -0.5 0.5) (end -0.5 -0.5) (stroke (width 0.15) (type solid)) (layer "F.SilkS"))
  (fp_rect (start -3.198439 -0.80055) (end -2.635868 0.799699) (stroke (width -0.000001) (type solid)) (fill yes) (layer "F.SilkS"))
  (fp_poly
   (pts (xy 3.19853 -0.800292) (xy -3.201338 -0.800292) (xy -3.201338 -0.651431) (xy -3.053026 -0.651431) (xy 3.050219 -0.651431)
    (xy 3.050219 0.649232) (xy -3.053026 0.649232) (xy -3.053026 -0.651431) (xy -3.201338 -0.651431) (xy -3.201338 0.800709)
    (xy 3.19853 0.800709))
   (stroke (width -0.000001) (type solid)) (fill yes) (layer "F.SilkS"))
  (pad "1" thru_hole rect (at -3.81 0 90) (size 1.397 1.397) (drill 0.8128) (layers "*.Cu" "*.Mask") (remove_unused_layers no)
   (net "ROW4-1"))
  (pad "1" smd rect (at -2.75 0 270) (size 2 0.5) (layers "F.Cu") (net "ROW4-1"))
  (pad "1" smd rect (at -2.75 0 90) (size 2 0.5) (layers "B.Cu") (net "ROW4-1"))
  (pad "1" smd rect (at -1.775 0 270) (size 1.4 0.94) (layers "F.Cu" "F.Mask" "F.Paste") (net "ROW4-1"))
  (pad "1" smd rect (at -1.775 0 90) (size 1.4 0.94) (layers "B.Cu" "B.Mask" "B.Paste") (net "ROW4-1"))
  (pad "2" smd rect (at 1.775 0 270) (size 1.4 0.94) (layers "F.Cu" "F.Mask" "F.Paste") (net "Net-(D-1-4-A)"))
  (pad "2" smd rect (at 1.775 0 90) (size 1.4 0.94) (layers "B.Cu" "B.Mask" "B.Paste") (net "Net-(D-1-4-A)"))
  (pad "2" smd rect (at 2.75 0 270) (size 2 0.5) (layers "F.Cu") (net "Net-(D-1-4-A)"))
  (pad "2" smd rect (at 2.75 0 90) (size 2 0.5) (layers "B.Cu") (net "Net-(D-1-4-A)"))
  (pad "2" thru_hole circle (at 3.81 0 90) (size 1.397 1.397) (drill 0.8128) (layers "*.Cu" "*.Mask") (remove_unused_layers no)
   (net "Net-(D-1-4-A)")))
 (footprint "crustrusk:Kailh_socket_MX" (layer "F.Cu") (at 89.549005 49.14 90)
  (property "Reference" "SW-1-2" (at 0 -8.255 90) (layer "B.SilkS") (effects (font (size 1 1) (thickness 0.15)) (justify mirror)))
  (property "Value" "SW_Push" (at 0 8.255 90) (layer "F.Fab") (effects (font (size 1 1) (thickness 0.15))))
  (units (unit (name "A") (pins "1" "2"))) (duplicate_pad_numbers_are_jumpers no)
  (fp_line (start 7 -7) (end 6 -7) (stroke (width 0.15) (type solid)) (layer "F.SilkS"))
  (fp_line (start 7 -7) (end 7 -6) (stroke (width 0.15) (type solid)) (layer "F.SilkS"))
  (fp_line (start -6 -7) (end -7 -7) (stroke (width 0.15) (type solid)) (layer "F.SilkS"))
  (fp_line (start -7 -6) (end -7 -7) (stroke (width 0.15) (type solid)) (layer "F.SilkS"))
  (fp_line (start 7 6) (end 7 7) (stroke (width 0.15) (type solid)) (layer "F.SilkS"))
  (fp_line (start 6 7) (end 7 7) (stroke (width 0.15) (type solid)) (layer "F.SilkS"))
  (fp_line (start -7 7) (end -7 6) (stroke (width 0.15) (type solid)) (layer "F.SilkS"))
  (fp_line (start -7 7) (end -6 7) (stroke (width 0.15) (type solid)) (layer "F.SilkS"))
  (pad "" np_thru_hole circle (at -5.08 0 90) (size 1.7018 1.7018) (drill 1.7018) (layers "*.Cu" "*.Mask"))
  (pad "" np_thru_hole circle (at -3.81 -2.54 90) (size 3 3) (drill 3) (layers "*.Cu" "*.Mask"))
  (pad "" np_thru_hole circle (at 0 0 90) (size 3.9878 3.9878) (drill 3.9878) (layers "*.Cu" "*.Mask"))
  (pad "" np_thru_hole circle (at 2.54 -5.08 90) (size 3 3) (drill 3) (layers "*.Cu" "*.Mask"))
  (pad "" np_thru_hole circle (at 5.08 0 90) (size 1.7018 1.7018) (drill 1.7018) (layers "*.Cu" "*.Mask"))
  (pad "1" smd rect (at 6.29 -5.08 90) (size 2.55 2.5) (layers "B.Cu" "B.Mask" "B.Paste") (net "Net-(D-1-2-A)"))
  (pad "2" smd rect (at -7.56 -2.54 90) (size 2.55 2.5) (layers "B.Cu" "B.Mask" "B.Paste") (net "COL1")))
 (gr_line (start 34.4 41.1) (end 34.4 58.599958) (stroke (width 0.05) (type default)) (layer "Edge.Cuts"))
 (gr_line (start 135.15 41) (end 34.4 41.1) (stroke (width 0.05) (type default)) (layer "Edge.Cuts"))
 (gr_line (start 135.15 58.6) (end 34.4 58.599945) (stroke (width 0.05) (type default)) (layer "Edge.Cuts"))
 (gr_line (start 135.15 58.6) (end 135.15 41) (stroke (width 0.05) (type default)) (layer "Edge.Cuts"))
 (segment (start 39.994005 54.522792) (end 39.994005 45.325) (width 0.2) (layer "B.Cu") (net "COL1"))
 (segment (start 39.994005 45.325) (end 41.169005 44.15) (width 0.2) (layer "B.Cu") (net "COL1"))
 (segment (start 49.009005 56.7) (end 68.009005 56.7) (width 0.2) (layer "B.Cu") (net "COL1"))
 (segment (start 42.171213 56.7) (end 39.994005 54.522792) (width 0.2) (layer "B.Cu") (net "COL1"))
 (segment (start 87.009005 56.7) (end 106 56.7) (width 0.2) (layer "B.Cu") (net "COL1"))
 (segment (start 125.01 56.71) (end 106.01 56.71) (width 0.2) (layer "B.Cu") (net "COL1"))
 (segment (start 49.009005 56.7) (end 42.171213 56.7) (width 0.2) (layer "B.Cu") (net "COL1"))
 (segment (start 68.009005 56.7) (end 87.009005 56.7) (width 0.2) (layer "B.Cu") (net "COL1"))
 (segment (start 106 56.7) (end 106.01 56.71) (width 0.2) (layer "B.Cu") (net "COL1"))
 (segment (start 55.379005 52.99) (end 51.6653 52.99) (width 0.2) (layer "F.Cu") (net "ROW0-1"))
 (segment (start 51.6653 52.99) (end 47.1253 48.45) (width 0.2) (layer "F.Cu") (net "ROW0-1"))
 (segment (start 47.1253 48.45) (end 43.469005 48.45) (width 0.2) (layer "F.Cu") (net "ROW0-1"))
 (segment (start 43.469005 48.45) (end 41.169005 46.15) (width 0.2) (layer "F.Cu") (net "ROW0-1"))
 (segment (start 71.819005 55.55) (end 48.569005 55.55) (width 0.2) (layer "F.Cu") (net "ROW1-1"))
 (segment (start 48.569005 55.55) (end 41.169005 48.15) (width 0.2) (layer "F.Cu") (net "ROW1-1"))
 (segment (start 74.379005 52.99) (end 71.819005 55.55) (width 0.2) (layer "F.Cu") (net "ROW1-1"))
 (segment (start 90.419005 55.95) (end 46.969005 55.95) (width 0.2) (layer "F.Cu") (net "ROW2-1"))
 (segment (start 93.379005 52.99) (end 90.419005 55.95) (width 0.2) (layer "F.Cu") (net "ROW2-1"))
 (segment (start 46.969005 55.95) (end 41.169005 50.15) (width 0.2) (layer "F.Cu") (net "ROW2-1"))
 (segment (start 109.03 56.35) (end 45.369005 56.35) (width 0.2) (layer "F.Cu") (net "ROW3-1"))
 (segment (start 112.38 53) (end 109.03 56.35) (width 0.2) (layer "F.Cu") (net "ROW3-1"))
 (segment (start 45.369005 56.35) (end 41.169005 52.15) (width 0.2) (layer "F.Cu") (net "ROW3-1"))
 (segment (start 127.63 56.75) (end 43.769005 56.75) (width 0.2) (layer "F.Cu") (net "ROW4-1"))
 (segment (start 43.769005 56.75) (end 41.169005 54.15) (width 0.2) (layer "F.Cu") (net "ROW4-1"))
 (segment (start 131.38 53) (end 127.63 56.75) (width 0.2) (layer "F.Cu") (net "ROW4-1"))
 (segment (start 65.469005 42.85) (end 72.444005 42.85) (width 0.2) (layer "B.Cu") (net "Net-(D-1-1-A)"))
 (segment (start 72.444005 42.85) (end 74.379005 44.785) (width 0.2) (layer "B.Cu") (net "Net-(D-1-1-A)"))
 (segment (start 46.469005 42.85) (end 48.949005 45.33) (width 0.2) (layer "B.Cu") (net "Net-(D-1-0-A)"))
 (segment (start 48.949005 45.33) (end 55.339005 45.33) (width 0.2) (layer "B.Cu") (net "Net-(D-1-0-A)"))
 (segment (start 103.47 42.86) (end 109.86 42.86) (width 0.2) (layer "B.Cu") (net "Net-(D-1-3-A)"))
 (segment (start 109.86 42.86) (end 112.38 45.38) (width 0.2) (layer "B.Cu") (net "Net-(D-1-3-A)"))
 (segment (start 93.379005 44.77) (end 93.379005 45.37) (width 0.2) (layer "B.Cu") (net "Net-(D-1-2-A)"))
 (segment (start 91.459005 42.85) (end 93.379005 44.77) (width 0.2) (layer "B.Cu") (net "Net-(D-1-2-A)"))
 (segment (start 84.469005 42.85) (end 91.459005 42.85) (width 0.2) (layer "B.Cu") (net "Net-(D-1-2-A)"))
 (segment (start 131.38 45.38) (end 128.8691 42.8691) (width 0.2) (layer "B.Cu") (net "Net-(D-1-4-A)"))
 (segment (start 122.4791 42.8691) (end 122.47 42.86) (width 0.2) (layer "B.Cu") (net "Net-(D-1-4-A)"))
 (segment (start 128.8691 42.8691) (end 122.4791 42.8691) (width 0.2) (layer "B.Cu") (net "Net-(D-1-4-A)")))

